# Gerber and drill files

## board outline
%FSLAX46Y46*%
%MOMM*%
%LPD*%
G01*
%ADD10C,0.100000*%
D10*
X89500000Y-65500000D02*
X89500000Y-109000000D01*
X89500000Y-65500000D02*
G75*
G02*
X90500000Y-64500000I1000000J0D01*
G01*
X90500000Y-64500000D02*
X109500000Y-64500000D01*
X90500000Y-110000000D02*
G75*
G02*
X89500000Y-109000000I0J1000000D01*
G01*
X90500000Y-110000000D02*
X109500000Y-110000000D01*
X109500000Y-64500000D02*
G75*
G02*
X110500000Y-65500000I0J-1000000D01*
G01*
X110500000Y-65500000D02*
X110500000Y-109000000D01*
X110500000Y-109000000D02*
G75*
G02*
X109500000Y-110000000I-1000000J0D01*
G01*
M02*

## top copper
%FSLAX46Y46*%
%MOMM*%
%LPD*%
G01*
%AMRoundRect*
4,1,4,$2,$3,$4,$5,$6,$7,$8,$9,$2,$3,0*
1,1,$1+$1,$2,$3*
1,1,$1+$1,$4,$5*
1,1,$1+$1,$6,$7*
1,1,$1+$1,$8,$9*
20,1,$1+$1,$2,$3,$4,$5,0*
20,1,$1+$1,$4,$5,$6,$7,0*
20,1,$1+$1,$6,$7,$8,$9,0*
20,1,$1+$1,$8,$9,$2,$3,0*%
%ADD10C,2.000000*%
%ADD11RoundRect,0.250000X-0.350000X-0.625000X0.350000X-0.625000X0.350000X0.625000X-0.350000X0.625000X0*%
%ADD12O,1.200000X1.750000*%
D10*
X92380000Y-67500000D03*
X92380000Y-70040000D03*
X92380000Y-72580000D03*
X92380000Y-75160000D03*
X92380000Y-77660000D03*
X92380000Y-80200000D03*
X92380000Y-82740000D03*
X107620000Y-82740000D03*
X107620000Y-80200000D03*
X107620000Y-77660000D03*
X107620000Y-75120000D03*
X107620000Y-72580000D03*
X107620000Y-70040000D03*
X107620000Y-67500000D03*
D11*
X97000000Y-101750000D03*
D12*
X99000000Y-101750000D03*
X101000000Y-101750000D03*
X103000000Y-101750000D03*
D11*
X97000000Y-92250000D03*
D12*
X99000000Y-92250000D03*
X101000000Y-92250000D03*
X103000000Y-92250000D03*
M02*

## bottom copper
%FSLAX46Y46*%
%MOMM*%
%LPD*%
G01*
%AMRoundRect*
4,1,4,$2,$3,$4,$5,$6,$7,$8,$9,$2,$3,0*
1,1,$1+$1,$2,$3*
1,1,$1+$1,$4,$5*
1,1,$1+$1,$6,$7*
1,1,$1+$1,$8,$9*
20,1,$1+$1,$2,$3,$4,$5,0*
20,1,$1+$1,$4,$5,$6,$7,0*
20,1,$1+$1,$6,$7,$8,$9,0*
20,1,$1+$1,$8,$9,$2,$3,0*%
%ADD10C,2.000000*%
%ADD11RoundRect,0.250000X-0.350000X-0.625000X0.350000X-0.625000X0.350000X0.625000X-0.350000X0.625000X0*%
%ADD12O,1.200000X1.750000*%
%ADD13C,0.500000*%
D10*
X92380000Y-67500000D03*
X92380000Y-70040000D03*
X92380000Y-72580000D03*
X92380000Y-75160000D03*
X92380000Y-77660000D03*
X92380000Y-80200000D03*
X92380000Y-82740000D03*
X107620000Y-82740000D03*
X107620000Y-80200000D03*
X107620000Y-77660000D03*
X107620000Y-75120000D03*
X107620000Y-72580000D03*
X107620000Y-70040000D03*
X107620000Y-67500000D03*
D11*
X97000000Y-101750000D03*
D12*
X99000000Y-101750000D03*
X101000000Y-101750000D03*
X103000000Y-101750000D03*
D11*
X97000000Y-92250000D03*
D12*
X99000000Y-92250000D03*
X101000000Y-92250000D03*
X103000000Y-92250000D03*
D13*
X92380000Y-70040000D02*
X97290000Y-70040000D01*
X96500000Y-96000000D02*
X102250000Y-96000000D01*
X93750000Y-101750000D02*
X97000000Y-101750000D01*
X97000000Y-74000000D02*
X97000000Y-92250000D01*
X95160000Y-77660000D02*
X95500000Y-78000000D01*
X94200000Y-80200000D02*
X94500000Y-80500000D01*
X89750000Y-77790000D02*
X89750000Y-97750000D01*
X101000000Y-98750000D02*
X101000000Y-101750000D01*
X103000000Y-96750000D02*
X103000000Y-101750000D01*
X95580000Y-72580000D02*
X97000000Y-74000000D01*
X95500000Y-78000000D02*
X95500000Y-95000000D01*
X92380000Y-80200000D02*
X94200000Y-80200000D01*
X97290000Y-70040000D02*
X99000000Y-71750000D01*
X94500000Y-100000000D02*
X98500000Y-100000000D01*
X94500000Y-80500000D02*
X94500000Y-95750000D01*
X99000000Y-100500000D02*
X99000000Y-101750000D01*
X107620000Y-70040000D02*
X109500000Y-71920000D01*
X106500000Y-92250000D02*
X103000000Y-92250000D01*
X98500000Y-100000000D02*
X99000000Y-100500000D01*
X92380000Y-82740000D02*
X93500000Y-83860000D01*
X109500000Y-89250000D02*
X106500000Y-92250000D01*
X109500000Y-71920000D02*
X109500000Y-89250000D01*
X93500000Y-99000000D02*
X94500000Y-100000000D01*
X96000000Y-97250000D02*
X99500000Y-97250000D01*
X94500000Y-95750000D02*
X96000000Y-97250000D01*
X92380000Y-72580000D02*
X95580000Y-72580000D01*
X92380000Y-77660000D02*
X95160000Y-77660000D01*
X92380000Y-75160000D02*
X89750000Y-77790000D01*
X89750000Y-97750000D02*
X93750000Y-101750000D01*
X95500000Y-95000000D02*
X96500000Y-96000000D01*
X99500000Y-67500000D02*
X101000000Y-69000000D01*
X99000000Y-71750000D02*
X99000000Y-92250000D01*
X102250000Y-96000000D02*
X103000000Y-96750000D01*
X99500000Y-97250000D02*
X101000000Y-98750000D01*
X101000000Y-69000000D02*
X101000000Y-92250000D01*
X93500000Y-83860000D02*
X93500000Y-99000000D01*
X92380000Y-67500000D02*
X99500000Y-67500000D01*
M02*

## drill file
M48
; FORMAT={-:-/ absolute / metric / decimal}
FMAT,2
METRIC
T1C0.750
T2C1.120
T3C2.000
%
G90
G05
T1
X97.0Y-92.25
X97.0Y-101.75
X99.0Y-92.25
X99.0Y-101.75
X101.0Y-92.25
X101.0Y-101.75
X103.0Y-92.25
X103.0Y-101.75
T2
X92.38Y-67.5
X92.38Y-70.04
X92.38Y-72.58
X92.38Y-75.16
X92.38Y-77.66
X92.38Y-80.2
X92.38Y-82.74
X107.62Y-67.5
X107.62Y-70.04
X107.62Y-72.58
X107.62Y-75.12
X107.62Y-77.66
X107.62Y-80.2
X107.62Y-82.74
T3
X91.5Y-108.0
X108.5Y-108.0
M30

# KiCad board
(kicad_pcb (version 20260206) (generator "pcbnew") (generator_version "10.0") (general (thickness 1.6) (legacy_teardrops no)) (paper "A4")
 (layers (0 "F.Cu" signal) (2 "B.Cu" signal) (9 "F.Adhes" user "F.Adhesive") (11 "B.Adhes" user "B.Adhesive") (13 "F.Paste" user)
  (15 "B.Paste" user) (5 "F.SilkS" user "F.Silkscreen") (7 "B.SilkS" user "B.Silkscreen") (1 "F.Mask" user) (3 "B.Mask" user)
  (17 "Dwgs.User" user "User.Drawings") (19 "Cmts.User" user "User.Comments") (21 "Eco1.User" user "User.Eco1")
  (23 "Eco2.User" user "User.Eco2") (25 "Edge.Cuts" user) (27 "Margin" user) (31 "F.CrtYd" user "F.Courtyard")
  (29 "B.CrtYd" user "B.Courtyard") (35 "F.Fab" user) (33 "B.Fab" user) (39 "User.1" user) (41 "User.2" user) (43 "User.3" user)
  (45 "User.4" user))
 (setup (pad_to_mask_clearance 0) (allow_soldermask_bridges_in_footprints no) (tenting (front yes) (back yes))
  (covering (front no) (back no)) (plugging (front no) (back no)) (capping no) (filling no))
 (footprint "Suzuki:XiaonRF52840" (layer "F.Cu") (at 100 75.12 -90)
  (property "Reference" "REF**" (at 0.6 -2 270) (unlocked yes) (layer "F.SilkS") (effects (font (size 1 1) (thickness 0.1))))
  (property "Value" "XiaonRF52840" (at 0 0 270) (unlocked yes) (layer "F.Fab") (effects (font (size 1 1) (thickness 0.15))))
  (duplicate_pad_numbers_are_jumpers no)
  (pad "1" thru_hole circle (at -7.62 7.62 270) (size 2 2) (drill 1.12) (layers "*.Cu" "*.Mask") (remove_unused_layers no))
  (pad "2" thru_hole circle (at -5.08 7.62 270) (size 2 2) (drill 1.12) (layers "*.Cu" "*.Mask") (remove_unused_layers no))
  (pad "3" thru_hole circle (at -2.54 7.62 270) (size 2 2) (drill 1.12) (layers "*.Cu" "*.Mask") (remove_unused_layers no))
  (pad "4" thru_hole circle (at 0.04 7.62 270) (size 2 2) (drill 1.12) (layers "*.Cu" "*.Mask") (remove_unused_layers no))
  (pad "5" thru_hole circle (at 2.54 7.62 270) (size 2 2) (drill 1.12) (layers "*.Cu" "*.Mask") (remove_unused_layers no))
  (pad "6" thru_hole circle (at 5.08 7.62 270) (size 2 2) (drill 1.12) (layers "*.Cu" "*.Mask") (remove_unused_layers no))
  (pad "7" thru_hole circle (at 7.62 7.62 270) (size 2 2) (drill 1.12) (layers "*.Cu" "*.Mask") (remove_unused_layers no))
  (pad "8" thru_hole circle (at 7.62 -7.62 270) (size 2 2) (drill 1.12) (layers "*.Cu" "*.Mask") (remove_unused_layers no))
  (pad "9" thru_hole circle (at 5.08 -7.62 270) (size 2 2) (drill 1.12) (layers "*.Cu" "*.Mask") (remove_unused_layers no))
  (pad "10" thru_hole circle (at 2.54 -7.62 270) (size 2 2) (drill 1.12) (layers "*.Cu" "*.Mask") (remove_unused_layers no))
  (pad "11" thru_hole circle (at 0 -7.62 270) (size 2 2) (drill 1.12) (layers "*.Cu" "*.Mask") (remove_unused_layers no))
  (pad "12" thru_hole circle (at -2.54 -7.62 270) (size 2 2) (drill 1.12) (layers "*.Cu" "*.Mask") (remove_unused_layers no))
  (pad "13" thru_hole circle (at -5.08 -7.62 270) (size 2 2) (drill 1.12) (layers "*.Cu" "*.Mask") (remove_unused_layers no))
  (pad "14" thru_hole circle (at -7.62 -7.62 270) (size 2 2) (drill 1.12) (layers "*.Cu" "*.Mask") (remove_unused_layers no)))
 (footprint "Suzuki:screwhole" (layer "F.Cu") (at 108.75 108)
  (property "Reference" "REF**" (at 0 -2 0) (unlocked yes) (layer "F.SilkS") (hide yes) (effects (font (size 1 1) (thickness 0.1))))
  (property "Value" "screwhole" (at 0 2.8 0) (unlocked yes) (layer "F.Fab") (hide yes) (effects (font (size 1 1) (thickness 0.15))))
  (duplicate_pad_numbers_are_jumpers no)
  (pad "" np_thru_hole circle (at -0.25 0) (size 2 2) (drill 2) (layers "*.Cu" "*.Mask")))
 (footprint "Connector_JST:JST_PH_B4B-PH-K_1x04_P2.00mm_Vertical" (layer "F.Cu") (at 97 101.75)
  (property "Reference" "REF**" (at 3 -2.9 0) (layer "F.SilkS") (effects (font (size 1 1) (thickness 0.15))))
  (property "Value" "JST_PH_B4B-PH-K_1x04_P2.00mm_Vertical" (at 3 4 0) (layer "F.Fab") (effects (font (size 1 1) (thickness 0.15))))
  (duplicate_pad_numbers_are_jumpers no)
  (pad "1" thru_hole roundrect (at 0 0) (size 1.2 1.75) (drill 0.75) (layers "*.Cu" "*.Mask") (remove_unused_layers no)
   (roundrect_rratio 0.208333))
  (pad "2" thru_hole oval (at 2 0) (size 1.2 1.75) (drill 0.75) (layers "*.Cu" "*.Mask") (remove_unused_layers no))
  (pad "3" thru_hole oval (at 4 0) (size 1.2 1.75) (drill 0.75) (layers "*.Cu" "*.Mask") (remove_unused_layers no))
  (pad "4" thru_hole oval (at 6 0) (size 1.2 1.75) (drill 0.75) (layers "*.Cu" "*.Mask") (remove_unused_layers no)))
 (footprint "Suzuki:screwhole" (layer "F.Cu") (at 91.5 108)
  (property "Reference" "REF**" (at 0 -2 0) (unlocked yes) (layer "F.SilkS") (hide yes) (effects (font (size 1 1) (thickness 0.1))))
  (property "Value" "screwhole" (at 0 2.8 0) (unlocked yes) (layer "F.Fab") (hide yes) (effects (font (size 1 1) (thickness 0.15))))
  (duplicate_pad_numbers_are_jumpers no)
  (pad "" np_thru_hole circle (at 0 0) (size 2 2) (drill 2) (layers "*.Cu" "*.Mask")))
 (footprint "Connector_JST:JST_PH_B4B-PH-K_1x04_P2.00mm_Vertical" (layer "F.Cu") (at 97 92.25)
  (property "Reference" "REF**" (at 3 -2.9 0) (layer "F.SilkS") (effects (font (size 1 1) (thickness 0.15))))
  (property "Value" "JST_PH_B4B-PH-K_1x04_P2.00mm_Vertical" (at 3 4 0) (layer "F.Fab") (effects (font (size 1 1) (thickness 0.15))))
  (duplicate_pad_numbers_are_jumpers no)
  (pad "1" thru_hole roundrect (at 0 0) (size 1.2 1.75) (drill 0.75) (layers "*.Cu" "*.Mask") (remove_unused_layers no)
   (roundrect_rratio 0.208333))
  (pad "2" thru_hole oval (at 2 0) (size 1.2 1.75) (drill 0.75) (layers "*.Cu" "*.Mask") (remove_unused_layers no))
  (pad "3" thru_hole oval (at 4 0) (size 1.2 1.75) (drill 0.75) (layers "*.Cu" "*.Mask") (remove_unused_layers no))
  (pad "4" thru_hole oval (at 6 0) (size 1.2 1.75) (drill 0.75) (layers "*.Cu" "*.Mask") (remove_unused_layers no)))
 (gr_line (start 89.5 65.5) (end 89.5 109) (stroke (width 0.1) (type solid)) (layer "Edge.Cuts"))
 (gr_arc (start 89.5 65.5) (mid 89.792893 64.792893) (end 90.5 64.5) (stroke (width 0.1) (type default)) (layer "Edge.Cuts"))
 (gr_line (start 90.5 64.5) (end 109.5 64.5) (stroke (width 0.1) (type solid)) (layer "Edge.Cuts"))
 (gr_arc (start 90.5 110) (mid 89.792893 109.707107) (end 89.5 109) (stroke (width 0.1) (type default)) (layer "Edge.Cuts"))
 (gr_line (start 90.5 110) (end 109.5 110) (stroke (width 0.1) (type solid)) (layer "Edge.Cuts"))
 (gr_arc (start 109.5 64.5) (mid 110.207107 64.792893) (end 110.5 65.5) (stroke (width 0.1) (type default)) (layer "Edge.Cuts"))
 (gr_line (start 110.5 65.5) (end 110.5 109) (stroke (width 0.1) (type solid)) (layer "Edge.Cuts"))
 (gr_arc (start 110.5 109) (mid 110.207107 109.707107) (end 109.5 110) (stroke (width 0.1) (type default)) (layer "Edge.Cuts"))
 (segment (start 92.38 70.04) (end 97.29 70.04) (width 0.5) (layer "B.Cu") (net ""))
 (segment (start 96.5 96) (end 102.25 96) (width 0.5) (layer "B.Cu") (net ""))
 (segment (start 93.75 101.75) (end 97 101.75) (width 0.5) (layer "B.Cu") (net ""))
 (segment (start 97 74) (end 97 92.25) (width 0.5) (layer "B.Cu") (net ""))
 (segment (start 95.16 77.66) (end 95.5 78) (width 0.5) (layer "B.Cu") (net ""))
 (segment (start 94.2 80.2) (end 94.5 80.5) (width 0.5) (layer "B.Cu") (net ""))
 (segment (start 89.75 77.79) (end 89.75 97.75) (width 0.5) (layer "B.Cu") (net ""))
 (segment (start 101 98.75) (end 101 101.75) (width 0.5) (layer "B.Cu") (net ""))
 (segment (start 103 96.75) (end 103 101.75) (width 0.5) (layer "B.Cu") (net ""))
 (segment (start 95.58 72.58) (end 97 74) (width 0.5) (layer "B.Cu") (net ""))
 (segment (start 95.5 78) (end 95.5 95) (width 0.5) (layer "B.Cu") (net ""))
 (segment (start 92.38 80.2) (end 94.2 80.2) (width 0.5) (layer "B.Cu") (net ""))
 (segment (start 97.29 70.04) (end 99 71.75) (width 0.5) (layer "B.Cu") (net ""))
 (segment (start 94.5 100) (end 98.5 100) (width 0.5) (layer "B.Cu") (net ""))
 (segment (start 94.5 80.5) (end 94.5 95.75) (width 0.5) (layer "B.Cu") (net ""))
 (segment (start 99 100.5) (end 99 101.75) (width 0.5) (layer "B.Cu") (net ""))
 (segment (start 107.62 70.04) (end 109.5 71.92) (width 0.5) (layer "B.Cu") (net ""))
 (segment (start 106.5 92.25) (end 103 92.25) (width 0.5) (layer "B.Cu") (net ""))
 (segment (start 98.5 100) (end 99 100.5) (width 0.5) (layer "B.Cu") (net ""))
 (segment (start 92.38 82.74) (end 93.5 83.86) (width 0.5) (layer "B.Cu") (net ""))
 (segment (start 109.5 89.25) (end 106.5 92.25) (width 0.5) (layer "B.Cu") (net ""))
 (segment (start 109.5 71.92) (end 109.5 89.25) (width 0.5) (layer "B.Cu") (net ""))
 (segment (start 93.5 99) (end 94.5 100) (width 0.5) (layer "B.Cu") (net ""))
 (segment (start 96 97.25) (end 99.5 97.25) (width 0.5) (layer "B.Cu") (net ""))
 (segment (start 94.5 95.75) (end 96 97.25) (width 0.5) (layer "B.Cu") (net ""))
 (segment (start 92.38 72.58) (end 95.58 72.58) (width 0.5) (layer "B.Cu") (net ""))
 (segment (start 92.38 77.66) (end 95.16 77.66) (width 0.5) (layer "B.Cu") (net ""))
 (segment (start 92.38 75.16) (end 89.75 77.79) (width 0.5) (layer "B.Cu") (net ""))
 (segment (start 89.75 97.75) (end 93.75 101.75) (width 0.5) (layer "B.Cu") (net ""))
 (segment (start 95.5 95) (end 96.5 96) (width 0.5) (layer "B.Cu") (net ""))
 (segment (start 99.5 67.5) (end 101 69) (width 0.5) (layer "B.Cu") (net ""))
 (segment (start 99 71.75) (end 99 92.25) (width 0.5) (layer "B.Cu") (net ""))
 (segment (start 102.25 96) (end 103 96.75) (width 0.5) (layer "B.Cu") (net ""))
 (segment (start 99.5 97.25) (end 101 98.75) (width 0.5) (layer "B.Cu") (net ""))
 (segment (start 101 69) (end 101 92.25) (width 0.5) (layer "B.Cu") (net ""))
 (segment (start 93.5 83.86) (end 93.5 99) (width 0.5) (layer "B.Cu") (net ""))
 (segment (start 92.38 67.5) (end 99.5 67.5) (width 0.5) (layer "B.Cu") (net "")))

